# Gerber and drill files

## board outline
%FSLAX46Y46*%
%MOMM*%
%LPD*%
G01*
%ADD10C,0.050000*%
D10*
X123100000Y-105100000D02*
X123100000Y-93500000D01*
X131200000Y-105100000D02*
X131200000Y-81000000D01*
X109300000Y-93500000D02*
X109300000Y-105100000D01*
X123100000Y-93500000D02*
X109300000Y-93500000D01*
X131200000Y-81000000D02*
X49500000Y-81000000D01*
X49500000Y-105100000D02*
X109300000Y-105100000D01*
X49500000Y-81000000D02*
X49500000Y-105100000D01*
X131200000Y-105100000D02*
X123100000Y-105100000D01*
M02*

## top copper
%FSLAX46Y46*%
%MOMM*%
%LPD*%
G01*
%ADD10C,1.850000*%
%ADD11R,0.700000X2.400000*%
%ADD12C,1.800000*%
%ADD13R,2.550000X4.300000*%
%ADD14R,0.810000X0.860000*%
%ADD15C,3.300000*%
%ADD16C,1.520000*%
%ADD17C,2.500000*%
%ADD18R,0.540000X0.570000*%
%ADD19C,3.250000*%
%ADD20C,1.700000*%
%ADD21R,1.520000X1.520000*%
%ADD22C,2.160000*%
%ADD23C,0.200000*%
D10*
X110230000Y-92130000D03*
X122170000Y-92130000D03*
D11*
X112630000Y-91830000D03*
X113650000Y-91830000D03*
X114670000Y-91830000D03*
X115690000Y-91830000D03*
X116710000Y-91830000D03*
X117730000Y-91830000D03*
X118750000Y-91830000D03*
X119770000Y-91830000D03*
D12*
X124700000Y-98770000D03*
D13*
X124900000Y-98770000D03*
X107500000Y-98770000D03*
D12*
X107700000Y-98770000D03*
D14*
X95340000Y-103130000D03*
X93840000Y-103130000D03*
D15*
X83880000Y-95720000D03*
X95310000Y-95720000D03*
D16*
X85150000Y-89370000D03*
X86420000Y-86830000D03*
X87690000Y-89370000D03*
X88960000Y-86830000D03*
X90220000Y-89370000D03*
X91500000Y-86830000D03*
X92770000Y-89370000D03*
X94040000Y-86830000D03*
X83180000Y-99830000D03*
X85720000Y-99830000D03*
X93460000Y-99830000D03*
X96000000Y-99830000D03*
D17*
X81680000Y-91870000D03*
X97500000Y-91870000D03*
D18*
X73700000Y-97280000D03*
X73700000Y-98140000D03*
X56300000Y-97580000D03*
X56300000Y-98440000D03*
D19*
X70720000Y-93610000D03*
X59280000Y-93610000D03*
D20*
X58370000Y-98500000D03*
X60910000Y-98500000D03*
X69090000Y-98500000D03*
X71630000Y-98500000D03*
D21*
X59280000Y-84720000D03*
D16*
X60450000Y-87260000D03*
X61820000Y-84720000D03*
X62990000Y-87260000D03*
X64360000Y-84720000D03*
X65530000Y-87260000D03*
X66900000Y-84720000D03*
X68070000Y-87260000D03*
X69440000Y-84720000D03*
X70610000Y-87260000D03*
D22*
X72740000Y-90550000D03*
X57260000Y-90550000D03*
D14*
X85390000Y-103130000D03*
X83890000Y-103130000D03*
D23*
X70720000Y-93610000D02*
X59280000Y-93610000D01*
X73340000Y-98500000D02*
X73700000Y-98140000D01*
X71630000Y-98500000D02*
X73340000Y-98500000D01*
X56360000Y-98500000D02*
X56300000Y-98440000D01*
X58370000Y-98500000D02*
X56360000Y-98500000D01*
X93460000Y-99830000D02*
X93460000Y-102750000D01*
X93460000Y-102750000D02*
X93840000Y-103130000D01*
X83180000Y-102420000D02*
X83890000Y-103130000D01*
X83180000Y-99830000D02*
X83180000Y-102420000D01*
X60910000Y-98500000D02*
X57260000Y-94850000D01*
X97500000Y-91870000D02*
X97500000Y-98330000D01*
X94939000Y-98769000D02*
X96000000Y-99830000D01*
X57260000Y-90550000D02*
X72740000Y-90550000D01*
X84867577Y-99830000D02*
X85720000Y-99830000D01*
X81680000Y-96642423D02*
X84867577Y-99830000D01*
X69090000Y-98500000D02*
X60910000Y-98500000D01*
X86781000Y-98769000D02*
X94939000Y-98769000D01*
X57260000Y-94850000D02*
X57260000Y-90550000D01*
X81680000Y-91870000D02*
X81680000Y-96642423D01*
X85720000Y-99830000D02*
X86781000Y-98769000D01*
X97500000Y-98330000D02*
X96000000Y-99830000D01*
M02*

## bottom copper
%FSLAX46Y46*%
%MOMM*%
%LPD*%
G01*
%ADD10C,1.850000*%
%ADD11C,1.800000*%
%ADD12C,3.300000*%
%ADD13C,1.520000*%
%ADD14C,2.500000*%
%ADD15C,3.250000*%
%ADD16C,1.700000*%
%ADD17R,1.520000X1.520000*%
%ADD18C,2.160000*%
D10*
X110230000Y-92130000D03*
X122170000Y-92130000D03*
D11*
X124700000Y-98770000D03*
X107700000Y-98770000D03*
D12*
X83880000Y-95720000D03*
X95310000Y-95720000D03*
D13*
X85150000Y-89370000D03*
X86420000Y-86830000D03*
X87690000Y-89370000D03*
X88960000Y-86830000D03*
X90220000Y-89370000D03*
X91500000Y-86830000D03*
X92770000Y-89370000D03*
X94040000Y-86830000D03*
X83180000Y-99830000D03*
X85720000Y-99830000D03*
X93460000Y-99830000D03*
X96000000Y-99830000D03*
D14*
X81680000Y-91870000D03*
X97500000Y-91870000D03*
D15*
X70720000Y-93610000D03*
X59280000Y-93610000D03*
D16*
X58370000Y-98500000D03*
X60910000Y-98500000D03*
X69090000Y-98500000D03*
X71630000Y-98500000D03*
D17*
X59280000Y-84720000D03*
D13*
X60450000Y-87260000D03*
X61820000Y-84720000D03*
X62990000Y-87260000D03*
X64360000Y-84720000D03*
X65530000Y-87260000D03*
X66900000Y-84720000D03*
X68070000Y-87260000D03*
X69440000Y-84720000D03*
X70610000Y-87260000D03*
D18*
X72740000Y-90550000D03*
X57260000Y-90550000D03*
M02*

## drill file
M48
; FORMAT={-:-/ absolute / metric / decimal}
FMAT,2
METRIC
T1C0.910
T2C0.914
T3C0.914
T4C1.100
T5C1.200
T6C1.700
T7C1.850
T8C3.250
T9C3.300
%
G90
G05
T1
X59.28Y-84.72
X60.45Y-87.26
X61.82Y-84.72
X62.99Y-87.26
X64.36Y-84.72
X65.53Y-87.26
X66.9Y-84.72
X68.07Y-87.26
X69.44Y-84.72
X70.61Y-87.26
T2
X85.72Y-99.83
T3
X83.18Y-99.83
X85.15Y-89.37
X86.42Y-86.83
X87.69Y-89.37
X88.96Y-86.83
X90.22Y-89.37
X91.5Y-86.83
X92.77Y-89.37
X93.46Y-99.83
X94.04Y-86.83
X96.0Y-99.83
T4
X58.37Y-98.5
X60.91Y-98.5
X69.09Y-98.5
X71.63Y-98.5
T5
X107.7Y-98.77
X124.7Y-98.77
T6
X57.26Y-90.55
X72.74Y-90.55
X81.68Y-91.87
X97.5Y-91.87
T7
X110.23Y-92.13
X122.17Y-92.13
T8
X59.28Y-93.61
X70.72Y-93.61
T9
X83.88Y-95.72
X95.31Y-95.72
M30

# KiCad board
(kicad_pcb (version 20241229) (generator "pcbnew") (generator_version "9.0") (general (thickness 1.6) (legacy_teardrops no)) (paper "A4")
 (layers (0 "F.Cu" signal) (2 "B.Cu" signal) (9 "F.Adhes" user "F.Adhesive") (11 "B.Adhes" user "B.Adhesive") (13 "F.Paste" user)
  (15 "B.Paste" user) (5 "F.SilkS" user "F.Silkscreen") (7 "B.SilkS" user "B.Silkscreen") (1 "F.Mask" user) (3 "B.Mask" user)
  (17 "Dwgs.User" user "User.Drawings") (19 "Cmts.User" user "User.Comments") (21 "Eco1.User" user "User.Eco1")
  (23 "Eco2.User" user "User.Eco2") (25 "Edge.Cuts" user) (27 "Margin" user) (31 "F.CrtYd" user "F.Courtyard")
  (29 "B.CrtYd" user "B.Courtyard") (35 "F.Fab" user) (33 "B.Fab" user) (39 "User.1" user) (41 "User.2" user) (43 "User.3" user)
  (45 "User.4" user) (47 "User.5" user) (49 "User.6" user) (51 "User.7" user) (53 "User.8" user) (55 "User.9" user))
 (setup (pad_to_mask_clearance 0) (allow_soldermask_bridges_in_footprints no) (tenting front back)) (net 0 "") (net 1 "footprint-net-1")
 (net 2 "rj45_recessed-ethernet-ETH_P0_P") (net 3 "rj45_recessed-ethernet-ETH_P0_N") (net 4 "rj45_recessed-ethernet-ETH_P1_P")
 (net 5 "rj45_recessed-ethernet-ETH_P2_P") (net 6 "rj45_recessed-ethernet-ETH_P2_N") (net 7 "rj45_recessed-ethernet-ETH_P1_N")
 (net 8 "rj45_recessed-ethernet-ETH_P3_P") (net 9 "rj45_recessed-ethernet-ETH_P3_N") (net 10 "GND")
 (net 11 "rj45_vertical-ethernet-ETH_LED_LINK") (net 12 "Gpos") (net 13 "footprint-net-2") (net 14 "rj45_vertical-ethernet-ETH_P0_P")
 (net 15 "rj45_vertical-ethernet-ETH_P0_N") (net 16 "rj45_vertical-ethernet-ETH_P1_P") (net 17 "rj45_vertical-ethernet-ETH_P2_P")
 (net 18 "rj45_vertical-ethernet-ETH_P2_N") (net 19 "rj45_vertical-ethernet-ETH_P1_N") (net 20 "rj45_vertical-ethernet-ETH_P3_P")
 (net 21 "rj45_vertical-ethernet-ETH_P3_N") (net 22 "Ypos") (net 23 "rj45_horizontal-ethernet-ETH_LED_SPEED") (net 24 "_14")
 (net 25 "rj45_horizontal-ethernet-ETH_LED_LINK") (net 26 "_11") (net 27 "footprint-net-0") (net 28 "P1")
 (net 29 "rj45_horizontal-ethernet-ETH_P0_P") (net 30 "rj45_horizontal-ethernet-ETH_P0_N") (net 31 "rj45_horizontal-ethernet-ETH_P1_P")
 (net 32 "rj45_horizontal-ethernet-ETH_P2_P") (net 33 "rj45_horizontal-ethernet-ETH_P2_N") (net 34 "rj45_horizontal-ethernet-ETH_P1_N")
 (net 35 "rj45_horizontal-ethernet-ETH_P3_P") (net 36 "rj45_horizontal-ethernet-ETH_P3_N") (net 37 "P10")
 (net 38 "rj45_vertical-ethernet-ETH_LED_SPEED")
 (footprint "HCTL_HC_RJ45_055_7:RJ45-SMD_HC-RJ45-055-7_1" (layer "F.Cu") (at 116.2 95.3 0)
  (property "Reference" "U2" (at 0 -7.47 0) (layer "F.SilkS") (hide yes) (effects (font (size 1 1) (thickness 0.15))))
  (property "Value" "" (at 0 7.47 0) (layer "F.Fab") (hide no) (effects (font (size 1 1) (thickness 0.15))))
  (pad "" thru_hole circle (at -5.97 -3.17 0) (size 1.85 1.85) (drill 1.85) (layers "*.Cu" "*.Mask") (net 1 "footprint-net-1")
   (remove_unused_layers no))
  (pad "" thru_hole circle (at 5.97 -3.17 0) (size 1.85 1.85) (drill 1.85) (layers "*.Cu" "*.Mask") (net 1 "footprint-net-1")
   (remove_unused_layers no))
  (pad "1" smd rect (at -3.57 -3.47 0) (size 0.7 2.4) (layers "F.Cu" "F.Mask" "F.Paste") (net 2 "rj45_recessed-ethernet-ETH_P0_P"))
  (pad "2" smd rect (at -2.55 -3.47 0) (size 0.7 2.4) (layers "F.Cu" "F.Mask" "F.Paste") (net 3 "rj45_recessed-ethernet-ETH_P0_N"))
  (pad "3" smd rect (at -1.53 -3.47 0) (size 0.7 2.4) (layers "F.Cu" "F.Mask" "F.Paste") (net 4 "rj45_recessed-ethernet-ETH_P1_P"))
  (pad "4" smd rect (at -0.51 -3.47 0) (size 0.7 2.4) (layers "F.Cu" "F.Mask" "F.Paste") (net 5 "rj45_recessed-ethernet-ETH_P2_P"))
  (pad "5" smd rect (at 0.51 -3.47 0) (size 0.7 2.4) (layers "F.Cu" "F.Mask" "F.Paste") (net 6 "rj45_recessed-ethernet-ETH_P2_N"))
  (pad "6" smd rect (at 1.53 -3.47 0) (size 0.7 2.4) (layers "F.Cu" "F.Mask" "F.Paste") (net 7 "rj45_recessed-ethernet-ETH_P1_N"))
  (pad "7" smd rect (at 2.55 -3.47 0) (size 0.7 2.4) (layers "F.Cu" "F.Mask" "F.Paste") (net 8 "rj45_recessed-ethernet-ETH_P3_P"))
  (pad "8" smd rect (at 3.57 -3.47 0) (size 0.7 2.4) (layers "F.Cu" "F.Mask" "F.Paste") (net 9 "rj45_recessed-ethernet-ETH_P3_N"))
  (pad "9" thru_hole circle (at 8.5 3.47 0) (size 1.8 1.8) (drill 1.199998) (layers "*.Cu" "*.Mask") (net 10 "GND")
   (remove_unused_layers no))
  (pad "9" smd rect (at 8.7 3.47 0) (size 2.55 4.3) (layers "F.Cu" "F.Mask" "F.Paste") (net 10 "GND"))
  (pad "10" smd rect (at -8.7 3.47 0) (size 2.55 4.3) (layers "F.Cu" "F.Mask" "F.Paste") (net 10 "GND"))
  (pad "10" thru_hole circle (at -8.5 3.47 0) (size 1.8 1.8) (drill 1.199998) (layers "*.Cu" "*.Mask") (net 10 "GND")
   (remove_unused_layers no)))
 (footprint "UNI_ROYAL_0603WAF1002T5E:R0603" (layer "F.Cu") (at 94.59 103.13 180)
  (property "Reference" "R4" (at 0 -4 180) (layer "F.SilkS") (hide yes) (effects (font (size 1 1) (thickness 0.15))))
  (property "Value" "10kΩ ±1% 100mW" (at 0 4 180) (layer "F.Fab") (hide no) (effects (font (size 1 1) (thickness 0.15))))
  (pad "1" smd rect (at -0.75 0 180) (size 0.81 0.86) (layers "F.Cu" "F.Mask" "F.Paste") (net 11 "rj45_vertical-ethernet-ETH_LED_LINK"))
  (pad "2" smd rect (at 0.75 0 180) (size 0.81 0.86) (layers "F.Cu" "F.Mask" "F.Paste") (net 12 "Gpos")))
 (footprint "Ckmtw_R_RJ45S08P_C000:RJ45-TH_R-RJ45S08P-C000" (layer "F.Cu") (at 89.59 93.33 0)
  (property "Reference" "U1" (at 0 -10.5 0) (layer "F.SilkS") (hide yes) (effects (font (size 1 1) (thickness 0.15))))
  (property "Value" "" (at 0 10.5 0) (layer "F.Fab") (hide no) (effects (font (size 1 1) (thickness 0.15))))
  (pad "" thru_hole circle (at -5.71 2.39 0) (size 3.3 3.3) (drill 3.3) (layers "*.Cu" "*.Mask") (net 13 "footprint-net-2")
   (remove_unused_layers no))
  (pad "" thru_hole circle (at 5.72 2.39 0) (size 3.3 3.3) (drill 3.3) (layers "*.Cu" "*.Mask") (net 13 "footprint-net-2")
   (remove_unused_layers no))
  (pad "1" thru_hole circle (at -4.44 -3.96 0) (size 1.52 1.52) (drill 0.9144) (layers "*.Cu" "*.Mask")
   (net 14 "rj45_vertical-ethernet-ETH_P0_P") (remove_unused_layers no))
  (pad "2" thru_hole circle (at -3.17 -6.5 0) (size 1.52 1.52) (drill 0.9144) (layers "*.Cu" "*.Mask")
   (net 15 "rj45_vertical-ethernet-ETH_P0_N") (remove_unused_layers no))
  (pad "3" thru_hole circle (at -1.9 -3.96 0) (size 1.52 1.52) (drill 0.9144) (layers "*.Cu" "*.Mask")
   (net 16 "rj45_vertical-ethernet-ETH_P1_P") (remove_unused_layers no))
  (pad "4" thru_hole circle (at -0.63 -6.5 0) (size 1.52 1.52) (drill 0.9144) (layers "*.Cu" "*.Mask")
   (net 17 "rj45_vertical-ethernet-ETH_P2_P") (remove_unused_layers no))
  (pad "5" thru_hole circle (at 0.63 -3.96 0) (size 1.52 1.52) (drill 0.9144) (layers "*.Cu" "*.Mask")
   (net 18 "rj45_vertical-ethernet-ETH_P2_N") (remove_unused_layers no))
  (pad "6" thru_hole circle (at 1.91 -6.5 0) (size 1.52 1.52) (drill 0.9144) (layers "*.Cu" "*.Mask")
   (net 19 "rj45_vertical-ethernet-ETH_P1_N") (remove_unused_layers no))
  (pad "7" thru_hole circle (at 3.18 -3.96 0) (size 1.52 1.52) (drill 0.9144) (layers "*.Cu" "*.Mask")
   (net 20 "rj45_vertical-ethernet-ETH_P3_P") (remove_unused_layers no))
  (pad "8" thru_hole circle (at 4.45 -6.5 0) (size 1.52 1.52) (drill 0.9144) (layers "*.Cu" "*.Mask")
   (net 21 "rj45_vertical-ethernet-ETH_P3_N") (remove_unused_layers no))
  (pad "9" thru_hole circle (at -6.41 6.5 0) (size 1.52 1.52) (drill 0.9144) (layers "*.Cu" "*.Mask") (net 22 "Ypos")
   (remove_unused_layers no))
  (pad "10" thru_hole circle (at -3.87 6.5 0) (size 1.52 1.52) (drill 0.913994) (layers "*.Cu" "*.Mask") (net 10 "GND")
   (remove_unused_layers no))
  (pad "11" thru_hole circle (at 3.87 6.5 0) (size 1.52 1.52) (drill 0.9144) (layers "*.Cu" "*.Mask") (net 12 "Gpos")
   (remove_unused_layers no))
  (pad "12" thru_hole circle (at 6.41 6.5 0) (size 1.52 1.52) (drill 0.9144) (layers "*.Cu" "*.Mask") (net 10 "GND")
   (remove_unused_layers no))
  (pad "13" thru_hole circle (at -7.91 -1.46 0) (size 2.5 2.5) (drill 1.700022) (layers "*.Cu" "*.Mask") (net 10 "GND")
   (remove_unused_layers no))
  (pad "14" thru_hole circle (at 7.91 -1.46 0) (size 2.5 2.5) (drill 1.700022) (layers "*.Cu" "*.Mask") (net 10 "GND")
   (remove_unused_layers no)))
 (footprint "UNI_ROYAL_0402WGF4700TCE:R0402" (layer "F.Cu") (at 73.7 97.71 -90)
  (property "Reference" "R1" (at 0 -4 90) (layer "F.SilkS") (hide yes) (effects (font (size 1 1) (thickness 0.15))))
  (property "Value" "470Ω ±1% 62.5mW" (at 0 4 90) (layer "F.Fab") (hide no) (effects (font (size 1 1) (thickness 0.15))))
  (pad "1" smd rect (at -0.43 0 270) (size 0.57 0.54) (layers "F.Cu" "F.Mask" "F.Paste") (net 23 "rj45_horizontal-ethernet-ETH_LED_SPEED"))
  (pad "2" smd rect (at 0.43 0 270) (size 0.57 0.54) (layers "F.Cu" "F.Mask" "F.Paste") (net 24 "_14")))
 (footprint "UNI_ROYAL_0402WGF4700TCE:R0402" (layer "F.Cu") (at 56.3 98.01 -90)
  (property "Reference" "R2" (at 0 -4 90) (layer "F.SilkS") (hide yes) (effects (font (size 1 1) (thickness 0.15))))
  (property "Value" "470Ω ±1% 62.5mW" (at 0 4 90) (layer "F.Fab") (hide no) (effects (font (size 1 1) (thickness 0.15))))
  (pad "1" smd rect (at -0.43 0 270) (size 0.57 0.54) (layers "F.Cu" "F.Mask" "F.Paste") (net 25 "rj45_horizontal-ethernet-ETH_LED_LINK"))
  (pad "2" smd rect (at 0.43 0 270) (size 0.57 0.54) (layers "F.Cu" "F.Mask" "F.Paste") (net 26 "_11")))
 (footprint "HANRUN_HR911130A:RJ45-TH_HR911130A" (layer "F.Cu") (at 65 91.61 180)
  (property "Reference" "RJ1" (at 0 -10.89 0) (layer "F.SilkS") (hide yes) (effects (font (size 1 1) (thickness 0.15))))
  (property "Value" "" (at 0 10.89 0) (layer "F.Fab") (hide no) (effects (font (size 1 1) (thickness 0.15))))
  (pad "" thru_hole circle (at -5.72 -2 180) (size 3.25 3.25) (drill 3.25) (layers "*.Cu" "*.Mask") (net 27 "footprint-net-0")
   (remove_unused_layers no))
  (pad "" thru_hole circle (at 5.72 -2 180) (size 3.25 3.25) (drill 3.25) (layers "*.Cu" "*.Mask") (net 27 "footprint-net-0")
   (remove_unused_layers no))
  (pad "11" thru_hole circle (at 6.63 -6.89 0) (size 1.7 1.7) (drill 1.100023) (layers "*.Cu" "*.Mask") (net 26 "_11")
   (remove_unused_layers no))
  (pad "12" thru_hole circle (at 4.09 -6.89 0) (size 1.7 1.7) (drill 1.100023) (layers "*.Cu" "*.Mask") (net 10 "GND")
   (remove_unused_layers no))
  (pad "13" thru_hole circle (at -4.09 -6.89 0) (size 1.7 1.7) (drill 1.100023) (layers "*.Cu" "*.Mask") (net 10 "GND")
   (remove_unused_layers no))
  (pad "14" thru_hole circle (at -6.63 -6.89 0) (size 1.7 1.7) (drill 1.100023) (layers "*.Cu" "*.Mask") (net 24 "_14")
   (remove_unused_layers no))
  (pad "P1" thru_hole rect (at 5.72 6.89 0) (size 1.52 1.52) (drill 0.90998) (layers "*.Cu" "*.Mask") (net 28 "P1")
   (remove_unused_layers no))
  (pad "P2" thru_hole circle (at 4.55 4.35 0) (size 1.52 1.52) (drill 0.90998) (layers "*.Cu" "*.Mask")
   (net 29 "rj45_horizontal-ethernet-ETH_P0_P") (remove_unused_layers no))
  (pad "P3" thru_hole circle (at 3.18 6.89 0) (size 1.52 1.52) (drill 0.90998) (layers "*.Cu" "*.Mask")
   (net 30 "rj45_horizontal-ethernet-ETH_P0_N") (remove_unused_layers no))
  (pad "P4" thru_hole circle (at 2.01 4.35 0) (size 1.52 1.52) (drill 0.90998) (layers "*.Cu" "*.Mask")
   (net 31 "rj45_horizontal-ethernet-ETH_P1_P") (remove_unused_layers no))
  (pad "P5" thru_hole circle (at 0.64 6.89 0) (size 1.52 1.52) (drill 0.90998) (layers "*.Cu" "*.Mask")
   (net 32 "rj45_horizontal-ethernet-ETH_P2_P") (remove_unused_layers no))
  (pad "P6" thru_hole circle (at -0.53 4.35 0) (size 1.52 1.52) (drill 0.90998) (layers "*.Cu" "*.Mask")
   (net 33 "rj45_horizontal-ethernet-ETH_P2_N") (remove_unused_layers no))
  (pad "P7" thru_hole circle (at -1.9 6.89 0) (size 1.52 1.52) (drill 0.90998) (layers "*.Cu" "*.Mask")
   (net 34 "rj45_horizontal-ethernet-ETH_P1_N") (remove_unused_layers no))
  (pad "P8" thru_hole circle (at -3.07 4.35 0) (size 1.52 1.52) (drill 0.90998) (layers "*.Cu" "*.Mask")
   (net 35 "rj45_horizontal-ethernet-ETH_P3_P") (remove_unused_layers no))
  (pad "P9" thru_hole circle (at -4.44 6.89 0) (size 1.52 1.52) (drill 0.90998) (layers "*.Cu" "*.Mask")
   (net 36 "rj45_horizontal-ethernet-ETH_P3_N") (remove_unused_layers no))
  (pad "P10" thru_hole circle (at -5.61 4.35 0) (size 1.52 1.52) (drill 0.90998) (layers "*.Cu" "*.Mask") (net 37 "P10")
   (remove_unused_layers no))
  (pad "SHIELD0" thru_hole circle (at -7.74 1.06 0) (size 2.16 2.16) (drill 1.700022) (layers "*.Cu" "*.Mask") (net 10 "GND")
   (remove_unused_layers no))
  (pad "SHIELD1" thru_hole circle (at 7.74 1.06 0) (size 2.16 2.16) (drill 1.700022) (layers "*.Cu" "*.Mask") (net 10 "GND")
   (remove_unused_layers no)))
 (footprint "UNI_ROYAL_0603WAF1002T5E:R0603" (layer "F.Cu") (at 84.64 103.13 180)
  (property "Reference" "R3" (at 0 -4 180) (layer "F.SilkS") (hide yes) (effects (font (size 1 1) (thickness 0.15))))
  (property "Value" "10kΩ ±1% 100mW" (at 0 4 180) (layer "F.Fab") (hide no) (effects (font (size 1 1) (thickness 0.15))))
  (pad "1" smd rect (at -0.75 0 180) (size 0.81 0.86) (layers "F.Cu" "F.Mask" "F.Paste") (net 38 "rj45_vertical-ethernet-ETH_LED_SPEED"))
  (pad "2" smd rect (at 0.75 0 180) (size 0.81 0.86) (layers "F.Cu" "F.Mask" "F.Paste") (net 22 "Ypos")))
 (segment (start 70.72 93.61) (end 59.28 93.61) (width 0.2) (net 27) (layer "F.Cu"))
 (segment (start 73.34 98.5) (end 73.7 98.14) (width 0.2) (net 24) (layer "F.Cu"))
 (segment (start 71.63 98.5) (end 73.34 98.5) (width 0.2) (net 24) (layer "F.Cu"))
 (segment (start 56.36 98.5) (end 56.3 98.44) (width 0.2) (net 26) (layer "F.Cu"))
 (segment (start 58.37 98.5) (end 56.36 98.5) (width 0.2) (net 26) (layer "F.Cu"))
 (segment (start 93.46 99.83) (end 93.46 102.75) (width 0.2) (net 12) (layer "F.Cu"))
 (segment (start 93.46 102.75) (end 93.84 103.13) (width 0.2) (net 12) (layer "F.Cu"))
 (segment (start 83.18 102.42) (end 83.89 103.13) (width 0.2) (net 22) (layer "F.Cu"))
 (segment (start 83.18 99.83) (end 83.18 102.42) (width 0.2) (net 22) (layer "F.Cu"))
 (segment (start 60.91 98.5) (end 57.26 94.85) (width 0.2) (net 10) (layer "F.Cu"))
 (segment (start 97.5 91.87) (end 97.5 98.33) (width 0.2) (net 10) (layer "F.Cu"))
 (segment (start 94.939 98.769) (end 96 99.83) (width 0.2) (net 10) (layer "F.Cu"))
 (segment (start 57.26 90.55) (end 72.74 90.55) (width 0.2) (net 10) (layer "F.Cu"))
 (segment (start 84.867577 99.83) (end 85.72 99.83) (width 0.2) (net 10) (layer "F.Cu"))
 (segment (start 81.68 96.642423) (end 84.867577 99.83) (width 0.2) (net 10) (layer "F.Cu"))
 (segment (start 69.09 98.5) (end 60.91 98.5) (width 0.2) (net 10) (layer "F.Cu"))
 (segment (start 86.781 98.769) (end 94.939 98.769) (width 0.2) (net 10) (layer "F.Cu"))
 (segment (start 57.26 94.85) (end 57.26 90.55) (width 0.2) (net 10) (layer "F.Cu"))
 (segment (start 81.68 91.87) (end 81.68 96.642423) (width 0.2) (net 10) (layer "F.Cu"))
 (segment (start 85.72 99.83) (end 86.781 98.769) (width 0.2) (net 10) (layer "F.Cu"))
 (segment (start 97.5 98.33) (end 96 99.83) (width 0.2) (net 10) (layer "F.Cu"))
 (gr_line (start 123.1 105.1) (end 123.1 93.5) (stroke (width 0.05) (type default)) (layer "Edge.Cuts"))
 (gr_line (start 131.2 105.1) (end 131.2 81) (stroke (width 0.05) (type default)) (layer "Edge.Cuts"))
 (gr_line (start 109.3 93.5) (end 109.3 105.1) (stroke (width 0.05) (type default)) (layer "Edge.Cuts"))
 (gr_line (start 123.1 93.5) (end 109.3 93.5) (stroke (width 0.05) (type default)) (layer "Edge.Cuts"))
 (gr_line (start 131.2 81) (end 49.5 81) (stroke (width 0.05) (type default)) (layer "Edge.Cuts"))
 (gr_line (start 49.5 105.1) (end 109.3 105.1) (stroke (width 0.05) (type default)) (layer "Edge.Cuts"))
 (gr_line (start 49.5 81) (end 49.5 105.1) (stroke (width 0.05) (type default)) (layer "Edge.Cuts"))
 (gr_line (start 131.2 105.1) (end 123.1 105.1) (stroke (width 0.05) (type default)) (layer "Edge.Cuts")))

